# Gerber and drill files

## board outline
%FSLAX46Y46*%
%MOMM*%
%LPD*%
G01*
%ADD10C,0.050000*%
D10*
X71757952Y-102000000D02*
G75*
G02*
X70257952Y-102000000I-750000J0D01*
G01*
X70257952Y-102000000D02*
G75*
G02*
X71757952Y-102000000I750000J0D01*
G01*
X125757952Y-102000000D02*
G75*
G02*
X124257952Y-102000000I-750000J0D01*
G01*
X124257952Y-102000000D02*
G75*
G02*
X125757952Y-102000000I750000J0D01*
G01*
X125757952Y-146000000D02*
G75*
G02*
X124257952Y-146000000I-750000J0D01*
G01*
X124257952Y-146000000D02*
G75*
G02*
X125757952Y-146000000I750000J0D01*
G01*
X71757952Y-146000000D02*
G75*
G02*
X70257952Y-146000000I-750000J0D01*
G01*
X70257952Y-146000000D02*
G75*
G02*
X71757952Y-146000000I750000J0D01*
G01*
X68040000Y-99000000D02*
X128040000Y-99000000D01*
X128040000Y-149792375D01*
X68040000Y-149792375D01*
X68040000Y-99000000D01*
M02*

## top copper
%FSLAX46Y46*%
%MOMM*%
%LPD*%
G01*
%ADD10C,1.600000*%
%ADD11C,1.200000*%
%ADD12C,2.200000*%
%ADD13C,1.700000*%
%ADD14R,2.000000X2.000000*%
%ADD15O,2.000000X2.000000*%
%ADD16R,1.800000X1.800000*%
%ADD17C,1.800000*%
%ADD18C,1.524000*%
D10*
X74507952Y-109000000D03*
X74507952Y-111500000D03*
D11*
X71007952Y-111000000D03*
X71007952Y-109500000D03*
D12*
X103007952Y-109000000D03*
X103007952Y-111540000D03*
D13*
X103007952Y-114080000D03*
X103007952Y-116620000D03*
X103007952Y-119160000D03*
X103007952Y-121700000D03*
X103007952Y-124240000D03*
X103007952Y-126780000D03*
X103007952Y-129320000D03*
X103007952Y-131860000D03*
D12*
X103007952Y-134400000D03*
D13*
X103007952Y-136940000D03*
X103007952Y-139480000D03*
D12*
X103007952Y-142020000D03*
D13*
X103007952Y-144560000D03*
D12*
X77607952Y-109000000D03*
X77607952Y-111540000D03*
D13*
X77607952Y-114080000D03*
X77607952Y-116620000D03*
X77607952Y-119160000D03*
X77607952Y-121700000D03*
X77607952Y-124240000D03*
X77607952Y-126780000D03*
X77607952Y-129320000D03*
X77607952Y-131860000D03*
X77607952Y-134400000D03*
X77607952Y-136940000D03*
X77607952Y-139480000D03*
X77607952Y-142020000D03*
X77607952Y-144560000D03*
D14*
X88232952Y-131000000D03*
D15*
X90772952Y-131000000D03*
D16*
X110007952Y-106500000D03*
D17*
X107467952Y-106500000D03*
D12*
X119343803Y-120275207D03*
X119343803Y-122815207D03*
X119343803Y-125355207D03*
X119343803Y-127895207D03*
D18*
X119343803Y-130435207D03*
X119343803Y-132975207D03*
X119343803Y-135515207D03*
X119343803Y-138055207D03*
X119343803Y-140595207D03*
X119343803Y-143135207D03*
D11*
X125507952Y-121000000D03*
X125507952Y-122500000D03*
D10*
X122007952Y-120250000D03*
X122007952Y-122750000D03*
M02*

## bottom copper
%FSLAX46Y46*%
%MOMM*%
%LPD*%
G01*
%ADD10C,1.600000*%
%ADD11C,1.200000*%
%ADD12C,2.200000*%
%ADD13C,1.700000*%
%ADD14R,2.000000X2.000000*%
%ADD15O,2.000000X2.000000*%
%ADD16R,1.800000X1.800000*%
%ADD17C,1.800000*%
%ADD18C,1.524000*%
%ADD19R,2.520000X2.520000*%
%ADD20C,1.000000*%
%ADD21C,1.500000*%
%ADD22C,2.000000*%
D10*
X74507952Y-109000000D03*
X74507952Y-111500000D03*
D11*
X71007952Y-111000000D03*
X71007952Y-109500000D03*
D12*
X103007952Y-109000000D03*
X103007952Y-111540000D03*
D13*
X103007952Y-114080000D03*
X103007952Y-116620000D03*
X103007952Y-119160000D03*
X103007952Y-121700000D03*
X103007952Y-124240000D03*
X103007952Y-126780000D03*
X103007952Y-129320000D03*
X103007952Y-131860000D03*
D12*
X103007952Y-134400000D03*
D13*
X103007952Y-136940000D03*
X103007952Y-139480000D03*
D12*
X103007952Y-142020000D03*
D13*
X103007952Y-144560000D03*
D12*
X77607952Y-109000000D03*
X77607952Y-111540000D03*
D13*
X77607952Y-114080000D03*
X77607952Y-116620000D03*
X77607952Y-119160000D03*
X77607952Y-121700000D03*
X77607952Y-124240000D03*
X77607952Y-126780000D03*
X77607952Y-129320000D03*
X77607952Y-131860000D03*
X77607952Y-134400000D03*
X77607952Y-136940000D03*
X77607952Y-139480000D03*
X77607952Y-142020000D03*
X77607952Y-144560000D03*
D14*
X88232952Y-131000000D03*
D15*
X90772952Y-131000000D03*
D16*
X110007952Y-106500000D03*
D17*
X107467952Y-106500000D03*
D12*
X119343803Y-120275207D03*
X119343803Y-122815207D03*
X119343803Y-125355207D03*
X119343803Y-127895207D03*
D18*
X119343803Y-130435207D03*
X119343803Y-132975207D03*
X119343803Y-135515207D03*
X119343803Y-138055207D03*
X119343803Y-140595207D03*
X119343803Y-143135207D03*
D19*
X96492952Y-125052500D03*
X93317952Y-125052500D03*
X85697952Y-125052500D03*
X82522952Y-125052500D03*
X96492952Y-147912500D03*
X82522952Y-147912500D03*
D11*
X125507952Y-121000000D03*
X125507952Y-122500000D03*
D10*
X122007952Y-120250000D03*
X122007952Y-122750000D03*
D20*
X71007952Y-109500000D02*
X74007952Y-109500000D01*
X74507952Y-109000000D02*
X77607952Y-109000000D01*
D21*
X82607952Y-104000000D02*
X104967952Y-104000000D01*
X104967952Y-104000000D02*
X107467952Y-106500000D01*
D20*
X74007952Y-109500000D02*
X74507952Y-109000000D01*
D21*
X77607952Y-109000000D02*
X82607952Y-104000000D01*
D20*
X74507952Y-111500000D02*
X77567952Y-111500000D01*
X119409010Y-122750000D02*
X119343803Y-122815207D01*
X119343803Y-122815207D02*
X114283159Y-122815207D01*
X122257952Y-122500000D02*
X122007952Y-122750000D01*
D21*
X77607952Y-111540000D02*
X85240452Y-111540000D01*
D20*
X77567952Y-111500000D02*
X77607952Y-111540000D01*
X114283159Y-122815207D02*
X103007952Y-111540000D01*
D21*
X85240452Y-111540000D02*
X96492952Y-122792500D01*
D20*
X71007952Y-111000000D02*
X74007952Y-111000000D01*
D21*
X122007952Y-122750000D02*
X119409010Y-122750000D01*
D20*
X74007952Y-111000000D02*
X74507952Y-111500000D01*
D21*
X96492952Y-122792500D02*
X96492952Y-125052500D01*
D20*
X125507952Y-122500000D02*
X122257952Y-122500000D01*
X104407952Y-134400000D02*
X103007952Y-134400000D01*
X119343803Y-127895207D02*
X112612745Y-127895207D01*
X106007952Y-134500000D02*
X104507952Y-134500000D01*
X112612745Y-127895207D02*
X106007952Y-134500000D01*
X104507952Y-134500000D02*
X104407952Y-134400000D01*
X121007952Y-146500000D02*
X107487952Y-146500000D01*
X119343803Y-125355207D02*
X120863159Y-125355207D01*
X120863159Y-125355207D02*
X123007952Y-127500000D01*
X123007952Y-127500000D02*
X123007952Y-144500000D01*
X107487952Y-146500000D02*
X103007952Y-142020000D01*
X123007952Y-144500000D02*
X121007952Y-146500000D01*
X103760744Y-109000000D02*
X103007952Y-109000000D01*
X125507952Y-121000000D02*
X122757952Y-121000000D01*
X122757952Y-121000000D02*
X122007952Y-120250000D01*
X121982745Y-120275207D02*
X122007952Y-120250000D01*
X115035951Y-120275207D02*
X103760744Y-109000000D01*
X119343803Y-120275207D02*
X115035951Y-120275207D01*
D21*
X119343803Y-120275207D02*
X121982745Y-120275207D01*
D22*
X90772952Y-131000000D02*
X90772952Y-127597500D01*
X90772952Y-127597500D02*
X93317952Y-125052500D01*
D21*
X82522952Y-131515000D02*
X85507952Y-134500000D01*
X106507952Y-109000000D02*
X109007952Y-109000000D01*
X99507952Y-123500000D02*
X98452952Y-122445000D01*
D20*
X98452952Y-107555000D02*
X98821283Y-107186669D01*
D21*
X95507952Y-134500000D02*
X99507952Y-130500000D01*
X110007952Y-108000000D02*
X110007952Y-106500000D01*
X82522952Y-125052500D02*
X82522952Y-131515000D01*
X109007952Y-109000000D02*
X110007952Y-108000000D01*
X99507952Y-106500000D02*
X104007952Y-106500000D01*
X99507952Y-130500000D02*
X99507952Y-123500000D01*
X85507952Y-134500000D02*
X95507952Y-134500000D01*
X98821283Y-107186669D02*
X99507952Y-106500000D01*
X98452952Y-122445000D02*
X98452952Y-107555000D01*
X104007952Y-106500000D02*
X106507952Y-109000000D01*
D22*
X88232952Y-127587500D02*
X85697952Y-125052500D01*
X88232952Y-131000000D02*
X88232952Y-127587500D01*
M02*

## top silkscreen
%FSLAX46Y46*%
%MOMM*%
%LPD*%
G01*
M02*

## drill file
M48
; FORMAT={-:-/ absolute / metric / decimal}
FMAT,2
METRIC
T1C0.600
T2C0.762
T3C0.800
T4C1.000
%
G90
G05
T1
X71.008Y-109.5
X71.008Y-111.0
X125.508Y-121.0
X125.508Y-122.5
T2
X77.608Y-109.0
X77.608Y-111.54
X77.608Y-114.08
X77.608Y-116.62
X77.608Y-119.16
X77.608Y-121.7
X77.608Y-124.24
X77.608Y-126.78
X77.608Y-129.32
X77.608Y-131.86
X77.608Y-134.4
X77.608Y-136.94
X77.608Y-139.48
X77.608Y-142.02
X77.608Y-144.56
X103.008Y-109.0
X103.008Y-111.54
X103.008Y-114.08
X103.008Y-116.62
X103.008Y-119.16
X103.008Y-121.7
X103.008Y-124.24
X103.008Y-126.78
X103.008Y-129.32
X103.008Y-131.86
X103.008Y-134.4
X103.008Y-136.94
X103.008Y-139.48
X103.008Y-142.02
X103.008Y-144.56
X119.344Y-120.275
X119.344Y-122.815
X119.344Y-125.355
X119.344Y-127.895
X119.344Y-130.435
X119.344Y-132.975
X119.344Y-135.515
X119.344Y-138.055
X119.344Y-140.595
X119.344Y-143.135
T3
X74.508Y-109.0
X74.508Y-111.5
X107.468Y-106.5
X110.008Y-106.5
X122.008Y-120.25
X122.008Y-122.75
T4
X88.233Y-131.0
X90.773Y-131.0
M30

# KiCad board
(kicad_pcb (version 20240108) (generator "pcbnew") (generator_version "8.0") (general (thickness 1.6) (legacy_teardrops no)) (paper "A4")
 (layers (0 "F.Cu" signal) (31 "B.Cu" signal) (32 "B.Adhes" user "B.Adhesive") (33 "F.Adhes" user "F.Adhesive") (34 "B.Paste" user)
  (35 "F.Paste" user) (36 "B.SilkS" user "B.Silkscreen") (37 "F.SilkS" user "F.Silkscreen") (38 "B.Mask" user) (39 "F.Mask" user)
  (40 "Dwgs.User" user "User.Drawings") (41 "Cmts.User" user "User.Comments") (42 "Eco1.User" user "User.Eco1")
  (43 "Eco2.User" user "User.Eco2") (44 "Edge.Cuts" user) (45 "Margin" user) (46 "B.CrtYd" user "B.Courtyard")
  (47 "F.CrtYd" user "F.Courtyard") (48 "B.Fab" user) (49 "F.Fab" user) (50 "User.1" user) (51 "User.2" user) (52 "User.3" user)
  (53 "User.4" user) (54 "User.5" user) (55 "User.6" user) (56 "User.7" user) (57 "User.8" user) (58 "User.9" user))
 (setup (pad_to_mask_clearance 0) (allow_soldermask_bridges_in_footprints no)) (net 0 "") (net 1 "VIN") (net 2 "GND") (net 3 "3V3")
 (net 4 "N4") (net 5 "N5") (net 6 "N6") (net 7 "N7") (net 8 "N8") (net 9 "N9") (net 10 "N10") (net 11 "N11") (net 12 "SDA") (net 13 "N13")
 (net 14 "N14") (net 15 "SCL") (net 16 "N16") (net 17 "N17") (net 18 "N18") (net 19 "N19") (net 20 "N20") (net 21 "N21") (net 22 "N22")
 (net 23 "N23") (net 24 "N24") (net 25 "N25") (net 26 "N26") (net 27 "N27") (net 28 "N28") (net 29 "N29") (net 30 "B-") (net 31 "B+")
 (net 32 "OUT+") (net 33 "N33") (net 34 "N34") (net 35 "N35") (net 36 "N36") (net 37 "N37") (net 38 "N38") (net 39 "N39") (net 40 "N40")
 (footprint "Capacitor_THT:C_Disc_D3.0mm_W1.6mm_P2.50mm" (layer "B.Cu") (at 74.507952 109 -90)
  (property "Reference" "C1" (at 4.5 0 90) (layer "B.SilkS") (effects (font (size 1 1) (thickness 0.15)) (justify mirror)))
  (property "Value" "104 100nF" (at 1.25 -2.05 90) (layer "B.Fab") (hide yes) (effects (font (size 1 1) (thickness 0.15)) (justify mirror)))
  (pad "1" thru_hole circle (at 0 0 270) (size 1.6 1.6) (drill 0.8) (layers "*.Cu" "*.Mask") (remove_unused_layers no) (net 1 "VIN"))
  (pad "2" thru_hole circle (at 2.5 0 270) (size 1.6 1.6) (drill 0.8) (layers "*.Cu" "*.Mask") (remove_unused_layers no) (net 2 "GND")))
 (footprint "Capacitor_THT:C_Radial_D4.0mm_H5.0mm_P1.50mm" (layer "B.Cu") (at 71.007952 109.5 -90)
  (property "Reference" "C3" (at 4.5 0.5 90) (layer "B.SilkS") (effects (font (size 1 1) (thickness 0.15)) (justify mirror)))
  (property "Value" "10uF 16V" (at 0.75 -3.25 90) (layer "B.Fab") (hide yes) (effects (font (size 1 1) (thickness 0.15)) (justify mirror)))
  (pad "2" thru_hole circle (at 1.5 0 270) (size 1.2 1.2) (drill 0.6) (layers "*.Cu" "*.Mask") (remove_unused_layers no) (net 2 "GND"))
  (pad "E" thru_hole circle (at 0 0 270) (size 1.2 1.2) (drill 0.6) (layers "*.Cu" "*.Mask") (remove_unused_layers no) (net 1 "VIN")))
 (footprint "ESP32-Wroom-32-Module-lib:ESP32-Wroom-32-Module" (layer "B.Cu") (at 103.007952 101.38 180)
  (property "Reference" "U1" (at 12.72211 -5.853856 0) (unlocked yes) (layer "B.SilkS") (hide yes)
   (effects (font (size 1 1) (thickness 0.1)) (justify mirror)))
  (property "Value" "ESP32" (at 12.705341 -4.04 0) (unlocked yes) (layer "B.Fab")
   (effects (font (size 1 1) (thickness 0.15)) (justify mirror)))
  (pad "1" thru_hole circle (at 0 -7.62 180) (size 2.2 2.2) (drill 0.762) (layers "*.Cu" "*.Mask") (remove_unused_layers no) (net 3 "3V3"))
  (pad "2" thru_hole circle (at 0 -10.16 180) (size 2.2 2.2) (drill 0.762) (layers "*.Cu" "*.Mask") (remove_unused_layers no) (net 2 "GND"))
  (pad "3" thru_hole circle (at 0 -12.7 180) (size 1.7 1.7) (drill 0.762) (layers "*.Cu" "*.Mask") (remove_unused_layers no) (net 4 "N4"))
  (pad "4" thru_hole circle (at 0 -15.24 180) (size 1.7 1.7) (drill 0.762) (layers "*.Cu" "*.Mask") (remove_unused_layers no) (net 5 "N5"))
  (pad "5" thru_hole circle (at 0 -17.78 180) (size 1.7 1.7) (drill 0.762) (layers "*.Cu" "*.Mask") (remove_unused_layers no) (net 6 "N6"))
  (pad "6" thru_hole circle (at 0 -20.32 180) (size 1.7 1.7) (drill 0.762) (layers "*.Cu" "*.Mask") (remove_unused_layers no) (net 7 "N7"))
  (pad "7" thru_hole circle (at 0 -22.86 180) (size 1.7 1.7) (drill 0.762) (layers "*.Cu" "*.Mask") (remove_unused_layers no) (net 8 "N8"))
  (pad "8" thru_hole circle (at 0 -25.4 180) (size 1.7 1.7) (drill 0.762) (layers "*.Cu" "*.Mask") (remove_unused_layers no) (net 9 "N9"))
  (pad "9" thru_hole circle (at 0 -27.94 180) (size 1.7 1.7) (drill 0.762) (layers "*.Cu" "*.Mask") (remove_unused_layers no) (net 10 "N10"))
  (pad "10" thru_hole circle (at 0 -30.48 180) (size 1.7 1.7) (drill 0.762) (layers "*.Cu" "*.Mask") (remove_unused_layers no)
   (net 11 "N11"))
  (pad "11" thru_hole circle (at 0 -33.02 180) (size 2.2 2.2) (drill 0.762) (layers "*.Cu" "*.Mask") (remove_unused_layers no)
   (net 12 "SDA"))
  (pad "12" thru_hole circle (at 0 -35.56 180) (size 1.7 1.7) (drill 0.762) (layers "*.Cu" "*.Mask") (remove_unused_layers no)
   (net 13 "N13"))
  (pad "13" thru_hole circle (at 0 -38.1 180) (size 1.7 1.7) (drill 0.762) (layers "*.Cu" "*.Mask") (remove_unused_layers no) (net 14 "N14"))
  (pad "14" thru_hole circle (at 0 -40.64 180) (size 2.2 2.2) (drill 0.762) (layers "*.Cu" "*.Mask") (remove_unused_layers no)
   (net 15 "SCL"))
  (pad "15" thru_hole circle (at 0 -43.18 180) (size 1.7 1.7) (drill 0.762) (layers "*.Cu" "*.Mask") (remove_unused_layers no)
   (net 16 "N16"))
  (pad "16" thru_hole circle (at 25.4 -7.62 180) (size 2.2 2.2) (drill 0.762) (layers "*.Cu" "*.Mask") (remove_unused_layers no)
   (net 1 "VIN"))
  (pad "17" thru_hole circle (at 25.4 -10.16 180) (size 2.2 2.2) (drill 0.762) (layers "*.Cu" "*.Mask") (remove_unused_layers no)
   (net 2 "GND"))
  (pad "18" thru_hole circle (at 25.4 -12.7 180) (size 1.7 1.7) (drill 0.762) (layers "*.Cu" "*.Mask") (remove_unused_layers no)
   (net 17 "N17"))
  (pad "19" thru_hole circle (at 25.4 -15.24 180) (size 1.7 1.7) (drill 0.762) (layers "*.Cu" "*.Mask") (remove_unused_layers no)
   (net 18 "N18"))
  (pad "20" thru_hole circle (at 25.4 -17.78 180) (size 1.7 1.7) (drill 0.762) (layers "*.Cu" "*.Mask") (remove_unused_layers no)
   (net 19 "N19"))
  (pad "21" thru_hole circle (at 25.4 -20.32 180) (size 1.7 1.7) (drill 0.762) (layers "*.Cu" "*.Mask") (remove_unused_layers no)
   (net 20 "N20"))
  (pad "22" thru_hole circle (at 25.4 -22.86 180) (size 1.7 1.7) (drill 0.762) (layers "*.Cu" "*.Mask") (remove_unused_layers no)
   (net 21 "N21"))
  (pad "23" thru_hole circle (at 25.4 -25.4 180) (size 1.7 1.7) (drill 0.762) (layers "*.Cu" "*.Mask") (remove_unused_layers no)
   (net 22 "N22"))
  (pad "24" thru_hole circle (at 25.4 -27.94 180) (size 1.7 1.7) (drill 0.762) (layers "*.Cu" "*.Mask") (remove_unused_layers no)
   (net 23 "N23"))
  (pad "25" thru_hole circle (at 25.4 -30.48 180) (size 1.7 1.7) (drill 0.762) (layers "*.Cu" "*.Mask") (remove_unused_layers no)
   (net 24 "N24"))
  (pad "26" thru_hole circle (at 25.4 -33.02 180) (size 1.7 1.7) (drill 0.762) (layers "*.Cu" "*.Mask") (remove_unused_layers no)
   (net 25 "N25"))
  (pad "27" thru_hole circle (at 25.4 -35.56 180) (size 1.7 1.7) (drill 0.762) (layers "*.Cu" "*.Mask") (remove_unused_layers no)
   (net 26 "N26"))
  (pad "28" thru_hole circle (at 25.4 -38.1 180) (size 1.7 1.7) (drill 0.762) (layers "*.Cu" "*.Mask") (remove_unused_layers no)
   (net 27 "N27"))
  (pad "29" thru_hole circle (at 25.4 -40.64 180) (size 1.7 1.7) (drill 0.762) (layers "*.Cu" "*.Mask") (remove_unused_layers no)
   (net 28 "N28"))
  (pad "30" thru_hole circle (at 25.4 -43.18 180) (size 1.7 1.7) (drill 0.762) (layers "*.Cu" "*.Mask") (remove_unused_layers no)
   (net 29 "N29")))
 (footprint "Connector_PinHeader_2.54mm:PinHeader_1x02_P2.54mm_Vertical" (layer "B.Cu") (at 88.232952 131 -90)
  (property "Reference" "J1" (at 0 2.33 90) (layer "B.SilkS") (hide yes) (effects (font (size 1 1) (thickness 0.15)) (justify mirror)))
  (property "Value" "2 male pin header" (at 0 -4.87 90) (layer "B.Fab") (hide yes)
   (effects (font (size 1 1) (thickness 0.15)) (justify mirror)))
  (pad "1" thru_hole rect (at 0 0 270) (size 2 2) (drill 1) (layers "*.Cu" "*.Mask") (remove_unused_layers no) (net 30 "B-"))
  (pad "2" thru_hole oval (at 0 -2.54 270) (size 2 2) (drill 1) (layers "*.Cu" "*.Mask") (remove_unused_layers no) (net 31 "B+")))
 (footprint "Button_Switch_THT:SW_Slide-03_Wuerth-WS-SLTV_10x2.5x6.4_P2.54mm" (layer "B.Cu") (at 110.007952 106.5)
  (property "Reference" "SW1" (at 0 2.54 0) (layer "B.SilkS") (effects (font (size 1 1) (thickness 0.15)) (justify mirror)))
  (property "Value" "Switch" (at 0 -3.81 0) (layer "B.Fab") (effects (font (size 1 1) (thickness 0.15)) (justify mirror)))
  (pad "1" thru_hole rect (at 0 0) (size 1.8 1.8) (drill 0.8) (layers "*.Cu" "*.Mask") (remove_unused_layers no) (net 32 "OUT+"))
  (pad "2" thru_hole circle (at -2.54 0) (size 1.8 1.8) (drill 0.8) (layers "*.Cu" "*.Mask") (remove_unused_layers no) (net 1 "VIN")))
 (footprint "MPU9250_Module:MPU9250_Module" (layer "B.Cu") (at 113.007952 114.5 180)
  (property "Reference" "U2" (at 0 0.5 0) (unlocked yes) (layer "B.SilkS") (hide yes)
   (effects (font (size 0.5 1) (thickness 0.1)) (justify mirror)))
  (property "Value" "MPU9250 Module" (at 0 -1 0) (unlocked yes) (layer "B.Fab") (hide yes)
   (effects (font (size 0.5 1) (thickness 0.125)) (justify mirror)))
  (pad "1" thru_hole circle (at -6.335851 -5.775207 180) (size 2.2 2.2) (drill 0.762) (layers "*.Cu" "*.Mask") (remove_unused_layers no)
   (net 3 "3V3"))
  (pad "2" thru_hole circle (at -6.335851 -8.315207 180) (size 2.2 2.2) (drill 0.762) (layers "*.Cu" "*.Mask") (remove_unused_layers no)
   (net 2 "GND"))
  (pad "3" thru_hole circle (at -6.335851 -10.855207 180) (size 2.2 2.2) (drill 0.762) (layers "*.Cu" "*.Mask") (remove_unused_layers no)
   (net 15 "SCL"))
  (pad "4" thru_hole circle (at -6.335851 -13.395207 180) (size 2.2 2.2) (drill 0.762) (layers "*.Cu" "*.Mask") (remove_unused_layers no)
   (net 12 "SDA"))
  (pad "5" thru_hole circle (at -6.335851 -15.935207 180) (size 1.524 1.524) (drill 0.762) (layers "*.Cu" "*.Mask")
   (remove_unused_layers no) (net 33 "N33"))
  (pad "6" thru_hole circle (at -6.335851 -18.475207 180) (size 1.524 1.524) (drill 0.762) (layers "*.Cu" "*.Mask")
   (remove_unused_layers no) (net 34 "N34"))
  (pad "7" thru_hole circle (at -6.335851 -21.015207 180) (size 1.524 1.524) (drill 0.762) (layers "*.Cu" "*.Mask")
   (remove_unused_layers no) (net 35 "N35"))
  (pad "8" thru_hole circle (at -6.335851 -23.555207 180) (size 1.524 1.524) (drill 0.762) (layers "*.Cu" "*.Mask")
   (remove_unused_layers no) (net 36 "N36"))
  (pad "9" thru_hole circle (at -6.335851 -26.095207 180) (size 1.524 1.524) (drill 0.762) (layers "*.Cu" "*.Mask")
   (remove_unused_layers no) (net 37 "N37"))
  (pad "10" thru_hole circle (at -6.335851 -28.635207 180) (size 1.524 1.524) (drill 0.762) (layers "*.Cu" "*.Mask")
   (remove_unused_layers no) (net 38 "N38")))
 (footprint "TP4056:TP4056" (layer "B.Cu") (at 89.507952 116.7475 180)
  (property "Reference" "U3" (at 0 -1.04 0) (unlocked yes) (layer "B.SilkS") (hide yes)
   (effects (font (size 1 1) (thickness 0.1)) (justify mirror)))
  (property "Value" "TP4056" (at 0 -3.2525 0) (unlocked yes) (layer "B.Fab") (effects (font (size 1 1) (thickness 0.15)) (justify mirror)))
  (pad "1" smd rect (at -6.985 -8.305 90) (size 2.52 2.52) (layers "B.Cu" "B.Paste" "B.Mask") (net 2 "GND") (thermal_bridge_angle 45))
  (pad "2" smd rect (at -3.81 -8.305 90) (size 2.52 2.52) (layers "B.Cu" "B.Paste" "B.Mask") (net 31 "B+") (thermal_bridge_angle 45))
  (pad "3" smd rect (at 3.81 -8.305 90) (size 2.52 2.52) (layers "B.Cu" "B.Paste" "B.Mask") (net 30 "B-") (thermal_bridge_angle 45))
  (pad "4" smd rect (at 6.985 -8.305 90) (size 2.52 2.52) (layers "B.Cu" "B.Paste" "B.Mask") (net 32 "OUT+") (thermal_bridge_angle 45))
  (pad "5" smd rect (at -6.985 -31.165 90) (size 2.52 2.52) (layers "B.Cu" "B.Paste" "B.Mask") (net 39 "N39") (thermal_bridge_angle 45))
  (pad "6" smd rect (at 6.985 -31.165 90) (size 2.52 2.52) (layers "B.Cu" "B.Paste" "B.Mask") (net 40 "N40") (thermal_bridge_angle 45)))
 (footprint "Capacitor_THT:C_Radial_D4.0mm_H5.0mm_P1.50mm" (layer "B.Cu") (at 125.507952 121 -90)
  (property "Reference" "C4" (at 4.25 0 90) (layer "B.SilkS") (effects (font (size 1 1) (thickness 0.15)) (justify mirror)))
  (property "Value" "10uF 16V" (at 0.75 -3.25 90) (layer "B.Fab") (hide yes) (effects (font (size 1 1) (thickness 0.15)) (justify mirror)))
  (pad "1" thru_hole circle (at 0 0 270) (size 1.2 1.2) (drill 0.6) (layers "*.Cu" "*.Mask") (remove_unused_layers no) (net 3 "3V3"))
  (pad "2" thru_hole circle (at 1.5 0 270) (size 1.2 1.2) (drill 0.6) (layers "*.Cu" "*.Mask") (remove_unused_layers no) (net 2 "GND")))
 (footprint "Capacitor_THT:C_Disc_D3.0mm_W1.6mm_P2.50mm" (layer "B.Cu") (at 122.007952 120.25 -90)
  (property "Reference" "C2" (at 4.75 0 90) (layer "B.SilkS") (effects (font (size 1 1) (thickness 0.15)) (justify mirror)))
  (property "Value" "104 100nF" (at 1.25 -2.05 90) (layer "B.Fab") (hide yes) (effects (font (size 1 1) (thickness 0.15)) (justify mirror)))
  (pad "1" thru_hole circle (at 0 0 270) (size 1.6 1.6) (drill 0.8) (layers "*.Cu" "*.Mask") (remove_unused_layers no) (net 3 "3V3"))
  (pad "2" thru_hole circle (at 2.5 0 270) (size 1.6 1.6) (drill 0.8) (layers "*.Cu" "*.Mask") (remove_unused_layers no) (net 2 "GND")))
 (gr_circle (center 71.007952 102) (end 70.257952 102) (stroke (width 0.05) (type default)) (fill none) (layer "Edge.Cuts"))
 (gr_circle (center 125.007952 102) (end 124.257952 102) (stroke (width 0.05) (type default)) (fill none) (layer "Edge.Cuts"))
 (gr_circle (center 125.007952 146) (end 124.257952 146) (stroke (width 0.05) (type default)) (fill none) (layer "Edge.Cuts"))
 (gr_circle (center 71.007952 146) (end 70.257952 146) (stroke (width 0.05) (type default)) (fill none) (layer "Edge.Cuts"))
 (gr_rect (start 68.04 99) (end 128.04 149.792375) (stroke (width 0.05) (type default)) (fill none) (layer "Edge.Cuts"))
 (segment (start 71.007952 109.5) (end 74.007952 109.5) (width 1) (layer "B.Cu") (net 1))
 (segment (start 74.507952 109) (end 77.607952 109) (width 1) (layer "B.Cu") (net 1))
 (segment (start 82.607952 104) (end 104.967952 104) (width 1.5) (layer "B.Cu") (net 1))
 (segment (start 104.967952 104) (end 107.467952 106.5) (width 1.5) (layer "B.Cu") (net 1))
 (segment (start 74.007952 109.5) (end 74.507952 109) (width 1) (layer "B.Cu") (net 1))
 (segment (start 77.607952 109) (end 82.607952 104) (width 1.5) (layer "B.Cu") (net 1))
 (segment (start 74.507952 111.5) (end 77.567952 111.5) (width 1) (layer "B.Cu") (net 2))
 (segment (start 119.40901 122.75) (end 119.343803 122.815207) (width 1) (layer "B.Cu") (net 2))
 (segment (start 119.343803 122.815207) (end 114.283159 122.815207) (width 1) (layer "B.Cu") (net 2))
 (segment (start 122.257952 122.5) (end 122.007952 122.75) (width 1) (layer "B.Cu") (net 2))
 (segment (start 77.607952 111.54) (end 85.240452 111.54) (width 1.5) (layer "B.Cu") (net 2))
 (segment (start 77.567952 111.5) (end 77.607952 111.54) (width 1) (layer "B.Cu") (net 2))
 (segment (start 114.283159 122.815207) (end 103.007952 111.54) (width 1) (layer "B.Cu") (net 2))
 (segment (start 85.240452 111.54) (end 96.492952 122.7925) (width 1.5) (layer "B.Cu") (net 2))
 (segment (start 71.007952 111) (end 74.007952 111) (width 1) (layer "B.Cu") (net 2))
 (segment (start 122.007952 122.75) (end 119.40901 122.75) (width 1.5) (layer "B.Cu") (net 2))
 (segment (start 74.007952 111) (end 74.507952 111.5) (width 1) (layer "B.Cu") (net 2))
 (segment (start 96.492952 122.7925) (end 96.492952 125.0525) (width 1.5) (layer "B.Cu") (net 2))
 (segment (start 125.507952 122.5) (end 122.257952 122.5) (width 1) (layer "B.Cu") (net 2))
 (segment (start 104.407952 134.4) (end 103.007952 134.4) (width 1) (layer "B.Cu") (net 12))
 (segment (start 119.343803 127.895207) (end 112.612745 127.895207) (width 1) (layer "B.Cu") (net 12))
 (segment (start 106.007952 134.5) (end 104.507952 134.5) (width 1) (layer "B.Cu") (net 12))
 (segment (start 112.612745 127.895207) (end 106.007952 134.5) (width 1) (layer "B.Cu") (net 12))
 (segment (start 104.507952 134.5) (end 104.407952 134.4) (width 1) (layer "B.Cu") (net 12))
 (segment (start 121.007952 146.5) (end 107.487952 146.5) (width 1) (layer "B.Cu") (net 15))
 (segment (start 119.343803 125.355207) (end 120.863159 125.355207) (width 1) (layer "B.Cu") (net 15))
 (segment (start 120.863159 125.355207) (end 123.007952 127.5) (width 1) (layer "B.Cu") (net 15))
 (segment (start 123.007952 127.5) (end 123.007952 144.5) (width 1) (layer "B.Cu") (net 15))
 (segment (start 107.487952 146.5) (end 103.007952 142.02) (width 1) (layer "B.Cu") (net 15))
 (segment (start 123.007952 144.5) (end 121.007952 146.5) (width 1) (layer "B.Cu") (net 15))
 (segment (start 103.760744 109) (end 103.007952 109) (width 1) (layer "B.Cu") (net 3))
 (segment (start 125.507952 121) (end 122.757952 121) (width 1) (layer "B.Cu") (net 3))
 (segment (start 122.757952 121) (end 122.007952 120.25) (width 1) (layer "B.Cu") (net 3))
 (segment (start 121.982745 120.275207) (end 122.007952 120.25) (width 1) (layer "B.Cu") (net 3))
 (segment (start 115.035951 120.275207) (end 103.760744 109) (width 1) (layer "B.Cu") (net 3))
 (segment (start 119.343803 120.275207) (end 115.035951 120.275207) (width 1) (layer "B.Cu") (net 3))
 (segment (start 119.343803 120.275207) (end 121.982745 120.275207) (width 1.5) (layer "B.Cu") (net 3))
 (segment (start 90.772952 131) (end 90.772952 127.5975) (width 2) (layer "B.Cu") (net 31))
 (segment (start 90.772952 127.5975) (end 93.317952 125.0525) (width 2) (layer "B.Cu") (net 31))
 (segment (start 82.522952 131.515) (end 85.507952 134.5) (width 1.5) (layer "B.Cu") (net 32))
 (segment (start 106.507952 109) (end 109.007952 109) (width 1.5) (layer "B.Cu") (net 32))
 (segment (start 99.507952 123.5) (end 98.452952 122.445) (width 1.5) (layer "B.Cu") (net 32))
 (segment (start 98.452952 107.555) (end 98.821283 107.186669) (width 1) (layer "B.Cu") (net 32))
 (segment (start 95.507952 134.5) (end 99.507952 130.5) (width 1.5) (layer "B.Cu") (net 32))
 (segment (start 110.007952 108) (end 110.007952 106.5) (width 1.5) (layer "B.Cu") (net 32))
 (segment (start 82.522952 125.0525) (end 82.522952 131.515) (width 1.5) (layer "B.Cu") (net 32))
 (segment (start 109.007952 109) (end 110.007952 108) (width 1.5) (layer "B.Cu") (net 32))
 (segment (start 99.507952 106.5) (end 104.007952 106.5) (width 1.5) (layer "B.Cu") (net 32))
 (segment (start 99.507952 130.5) (end 99.507952 123.5) (width 1.5) (layer "B.Cu") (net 32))
 (segment (start 85.507952 134.5) (end 95.507952 134.5) (width 1.5) (layer "B.Cu") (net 32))
 (segment (start 98.821283 107.186669) (end 99.507952 106.5) (width 1.5) (layer "B.Cu") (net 32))
 (segment (start 98.452952 122.445) (end 98.452952 107.555) (width 1.5) (layer "B.Cu") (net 32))
 (segment (start 104.007952 106.5) (end 106.507952 109) (width 1.5) (layer "B.Cu") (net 32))
 (segment (start 88.232952 127.5875) (end 85.697952 125.0525) (width 2) (layer "B.Cu") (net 30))
 (segment (start 88.232952 131) (end 88.232952 127.5875) (width 2) (layer "B.Cu") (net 30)))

